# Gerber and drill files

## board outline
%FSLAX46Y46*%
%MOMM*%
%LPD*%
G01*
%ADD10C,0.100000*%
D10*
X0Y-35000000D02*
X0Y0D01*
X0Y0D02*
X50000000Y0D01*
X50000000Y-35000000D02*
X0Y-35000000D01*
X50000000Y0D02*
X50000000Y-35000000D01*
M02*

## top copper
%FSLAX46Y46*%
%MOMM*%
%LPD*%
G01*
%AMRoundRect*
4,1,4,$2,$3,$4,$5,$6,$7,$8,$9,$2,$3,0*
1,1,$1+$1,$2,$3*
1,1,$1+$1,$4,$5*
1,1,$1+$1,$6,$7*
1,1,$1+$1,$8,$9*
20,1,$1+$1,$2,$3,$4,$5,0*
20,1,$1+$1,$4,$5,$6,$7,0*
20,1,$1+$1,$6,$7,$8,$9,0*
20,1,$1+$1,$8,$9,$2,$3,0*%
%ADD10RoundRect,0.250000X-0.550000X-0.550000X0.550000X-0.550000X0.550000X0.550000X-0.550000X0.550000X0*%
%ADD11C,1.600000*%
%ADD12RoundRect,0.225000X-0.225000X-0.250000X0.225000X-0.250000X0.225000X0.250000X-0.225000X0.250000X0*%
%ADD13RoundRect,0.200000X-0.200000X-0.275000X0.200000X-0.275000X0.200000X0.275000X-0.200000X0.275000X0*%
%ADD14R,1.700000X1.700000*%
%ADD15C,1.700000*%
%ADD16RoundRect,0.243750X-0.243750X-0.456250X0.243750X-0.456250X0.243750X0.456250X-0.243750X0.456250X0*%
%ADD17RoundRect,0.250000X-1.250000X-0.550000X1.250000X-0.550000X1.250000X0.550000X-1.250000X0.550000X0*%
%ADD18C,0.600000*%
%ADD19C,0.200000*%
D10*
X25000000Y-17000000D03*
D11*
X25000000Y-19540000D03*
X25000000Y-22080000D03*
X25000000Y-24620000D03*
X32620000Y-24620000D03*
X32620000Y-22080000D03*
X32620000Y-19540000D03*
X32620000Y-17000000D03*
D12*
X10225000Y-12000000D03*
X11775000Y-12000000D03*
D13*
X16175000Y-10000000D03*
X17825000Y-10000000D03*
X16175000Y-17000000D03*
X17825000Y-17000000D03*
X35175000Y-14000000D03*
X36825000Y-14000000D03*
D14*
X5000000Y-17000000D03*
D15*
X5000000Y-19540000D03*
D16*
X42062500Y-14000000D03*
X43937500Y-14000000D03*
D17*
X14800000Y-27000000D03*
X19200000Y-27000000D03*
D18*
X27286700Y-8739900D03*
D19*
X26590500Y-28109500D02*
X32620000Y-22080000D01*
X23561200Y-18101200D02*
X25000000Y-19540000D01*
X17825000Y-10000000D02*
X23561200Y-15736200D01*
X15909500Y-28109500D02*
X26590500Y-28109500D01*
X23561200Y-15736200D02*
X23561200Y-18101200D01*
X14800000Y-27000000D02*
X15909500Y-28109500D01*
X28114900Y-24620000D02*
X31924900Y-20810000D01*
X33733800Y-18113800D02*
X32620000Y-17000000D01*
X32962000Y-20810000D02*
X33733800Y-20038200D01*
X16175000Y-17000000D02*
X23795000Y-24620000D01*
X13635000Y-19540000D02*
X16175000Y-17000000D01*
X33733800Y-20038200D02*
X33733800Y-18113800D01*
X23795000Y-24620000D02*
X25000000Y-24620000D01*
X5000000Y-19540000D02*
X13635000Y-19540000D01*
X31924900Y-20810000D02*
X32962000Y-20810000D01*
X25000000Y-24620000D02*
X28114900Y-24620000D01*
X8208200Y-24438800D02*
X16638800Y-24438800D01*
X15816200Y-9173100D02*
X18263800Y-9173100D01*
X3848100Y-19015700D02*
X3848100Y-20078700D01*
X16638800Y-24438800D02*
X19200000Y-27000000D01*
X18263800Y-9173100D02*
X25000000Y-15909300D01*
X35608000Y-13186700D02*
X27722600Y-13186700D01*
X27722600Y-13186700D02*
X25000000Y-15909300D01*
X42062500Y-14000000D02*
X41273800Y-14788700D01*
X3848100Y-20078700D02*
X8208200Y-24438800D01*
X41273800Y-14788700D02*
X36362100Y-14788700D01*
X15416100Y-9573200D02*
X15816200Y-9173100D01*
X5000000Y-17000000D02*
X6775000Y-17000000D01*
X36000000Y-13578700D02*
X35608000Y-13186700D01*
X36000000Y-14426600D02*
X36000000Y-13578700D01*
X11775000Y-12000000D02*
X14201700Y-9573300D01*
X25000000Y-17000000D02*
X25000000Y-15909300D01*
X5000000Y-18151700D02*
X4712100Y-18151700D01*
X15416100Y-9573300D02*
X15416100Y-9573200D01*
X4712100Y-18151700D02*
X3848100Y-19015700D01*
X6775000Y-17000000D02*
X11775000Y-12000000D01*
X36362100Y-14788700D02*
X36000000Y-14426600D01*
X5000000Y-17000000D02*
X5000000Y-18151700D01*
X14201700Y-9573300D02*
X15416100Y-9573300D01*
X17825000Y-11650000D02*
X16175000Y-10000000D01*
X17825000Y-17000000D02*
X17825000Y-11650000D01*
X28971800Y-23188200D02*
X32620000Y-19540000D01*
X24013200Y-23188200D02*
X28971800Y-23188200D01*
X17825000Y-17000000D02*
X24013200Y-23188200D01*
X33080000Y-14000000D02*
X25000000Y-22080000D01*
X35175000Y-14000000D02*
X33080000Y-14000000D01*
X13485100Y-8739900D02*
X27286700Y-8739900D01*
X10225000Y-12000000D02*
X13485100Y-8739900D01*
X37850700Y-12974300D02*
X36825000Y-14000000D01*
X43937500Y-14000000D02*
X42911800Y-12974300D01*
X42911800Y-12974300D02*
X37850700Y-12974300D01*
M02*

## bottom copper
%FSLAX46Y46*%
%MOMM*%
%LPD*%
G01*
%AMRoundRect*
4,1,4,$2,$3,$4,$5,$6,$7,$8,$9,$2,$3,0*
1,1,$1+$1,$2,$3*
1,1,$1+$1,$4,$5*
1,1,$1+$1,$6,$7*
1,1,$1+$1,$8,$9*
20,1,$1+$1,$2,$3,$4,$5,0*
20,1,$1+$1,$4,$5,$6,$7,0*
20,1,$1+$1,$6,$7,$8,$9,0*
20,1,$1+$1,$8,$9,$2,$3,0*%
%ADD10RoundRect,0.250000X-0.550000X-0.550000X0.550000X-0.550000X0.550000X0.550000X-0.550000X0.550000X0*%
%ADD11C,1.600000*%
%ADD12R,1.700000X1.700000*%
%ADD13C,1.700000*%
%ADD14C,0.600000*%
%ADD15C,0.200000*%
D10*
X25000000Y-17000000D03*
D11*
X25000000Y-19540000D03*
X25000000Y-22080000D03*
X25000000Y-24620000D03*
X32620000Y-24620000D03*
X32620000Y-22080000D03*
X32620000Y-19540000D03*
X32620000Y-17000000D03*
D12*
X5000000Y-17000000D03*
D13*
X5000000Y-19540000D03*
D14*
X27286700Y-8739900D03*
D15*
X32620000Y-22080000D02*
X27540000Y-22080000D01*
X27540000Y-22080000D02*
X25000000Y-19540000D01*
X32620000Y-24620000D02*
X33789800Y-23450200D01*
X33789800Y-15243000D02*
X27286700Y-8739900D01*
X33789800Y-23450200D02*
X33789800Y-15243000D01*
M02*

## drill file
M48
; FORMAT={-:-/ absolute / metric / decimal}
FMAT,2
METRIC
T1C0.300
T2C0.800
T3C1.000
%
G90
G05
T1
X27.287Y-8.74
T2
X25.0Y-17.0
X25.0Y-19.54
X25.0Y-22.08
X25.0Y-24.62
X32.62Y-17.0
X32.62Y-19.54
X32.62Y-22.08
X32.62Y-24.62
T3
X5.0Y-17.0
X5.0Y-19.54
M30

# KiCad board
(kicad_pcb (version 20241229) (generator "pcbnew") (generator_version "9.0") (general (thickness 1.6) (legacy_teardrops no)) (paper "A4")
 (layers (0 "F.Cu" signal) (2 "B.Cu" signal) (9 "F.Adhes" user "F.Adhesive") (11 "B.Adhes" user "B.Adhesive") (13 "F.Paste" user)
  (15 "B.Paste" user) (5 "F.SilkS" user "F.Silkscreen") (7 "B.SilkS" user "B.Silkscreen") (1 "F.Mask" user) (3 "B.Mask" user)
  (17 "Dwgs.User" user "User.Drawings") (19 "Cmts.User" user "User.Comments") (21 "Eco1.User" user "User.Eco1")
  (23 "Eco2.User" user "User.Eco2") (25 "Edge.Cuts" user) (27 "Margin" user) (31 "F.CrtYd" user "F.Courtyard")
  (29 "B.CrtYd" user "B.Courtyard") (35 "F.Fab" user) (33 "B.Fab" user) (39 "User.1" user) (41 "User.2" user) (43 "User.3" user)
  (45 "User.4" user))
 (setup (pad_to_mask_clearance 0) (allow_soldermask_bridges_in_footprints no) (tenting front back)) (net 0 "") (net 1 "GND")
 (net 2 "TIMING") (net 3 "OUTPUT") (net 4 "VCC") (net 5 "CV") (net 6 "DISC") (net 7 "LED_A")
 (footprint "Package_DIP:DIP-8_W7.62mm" (layer "F.Cu") (at 25 17)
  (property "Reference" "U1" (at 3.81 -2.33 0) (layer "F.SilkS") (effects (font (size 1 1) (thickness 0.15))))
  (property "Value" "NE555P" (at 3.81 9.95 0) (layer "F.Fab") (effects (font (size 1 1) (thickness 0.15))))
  (pad "1" thru_hole roundrect (at 0 0) (size 1.6 1.6) (drill 0.8) (layers "*.Cu" "*.Mask") (remove_unused_layers no)
   (roundrect_rratio 0.15625) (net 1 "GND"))
  (pad "2" thru_hole circle (at 0 2.54) (size 1.6 1.6) (drill 0.8) (layers "*.Cu" "*.Mask") (remove_unused_layers no) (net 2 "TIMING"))
  (pad "3" thru_hole circle (at 0 5.08) (size 1.6 1.6) (drill 0.8) (layers "*.Cu" "*.Mask") (remove_unused_layers no) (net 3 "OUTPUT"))
  (pad "4" thru_hole circle (at 0 7.62) (size 1.6 1.6) (drill 0.8) (layers "*.Cu" "*.Mask") (remove_unused_layers no) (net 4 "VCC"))
  (pad "5" thru_hole circle (at 7.62 7.62) (size 1.6 1.6) (drill 0.8) (layers "*.Cu" "*.Mask") (remove_unused_layers no) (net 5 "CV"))
  (pad "6" thru_hole circle (at 7.62 5.08) (size 1.6 1.6) (drill 0.8) (layers "*.Cu" "*.Mask") (remove_unused_layers no) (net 2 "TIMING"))
  (pad "7" thru_hole circle (at 7.62 2.54) (size 1.6 1.6) (drill 0.8) (layers "*.Cu" "*.Mask") (remove_unused_layers no) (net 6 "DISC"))
  (pad "8" thru_hole circle (at 7.62 0) (size 1.6 1.6) (drill 0.8) (layers "*.Cu" "*.Mask") (remove_unused_layers no) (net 4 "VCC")))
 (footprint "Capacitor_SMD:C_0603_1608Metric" (layer "F.Cu") (at 11 12)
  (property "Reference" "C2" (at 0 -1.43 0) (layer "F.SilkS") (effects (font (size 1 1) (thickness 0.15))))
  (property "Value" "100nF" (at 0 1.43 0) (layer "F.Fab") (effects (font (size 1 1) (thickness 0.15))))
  (pad "1" smd roundrect (at -0.775 0) (size 0.9 0.95) (layers "F.Cu" "F.Mask" "F.Paste") (roundrect_rratio 0.25) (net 5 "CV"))
  (pad "2" smd roundrect (at 0.775 0) (size 0.9 0.95) (layers "F.Cu" "F.Mask" "F.Paste") (roundrect_rratio 0.25) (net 1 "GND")))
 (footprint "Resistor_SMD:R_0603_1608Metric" (layer "F.Cu") (at 17 10)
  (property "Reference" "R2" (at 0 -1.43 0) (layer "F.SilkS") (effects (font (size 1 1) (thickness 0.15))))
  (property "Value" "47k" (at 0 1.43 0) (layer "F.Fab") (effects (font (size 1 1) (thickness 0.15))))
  (pad "1" smd roundrect (at -0.825 0) (size 0.8 0.95) (layers "F.Cu" "F.Mask" "F.Paste") (roundrect_rratio 0.25) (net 6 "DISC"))
  (pad "2" smd roundrect (at 0.825 0) (size 0.8 0.95) (layers "F.Cu" "F.Mask" "F.Paste") (roundrect_rratio 0.25) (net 2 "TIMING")))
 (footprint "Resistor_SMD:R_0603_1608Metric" (layer "F.Cu") (at 17 17)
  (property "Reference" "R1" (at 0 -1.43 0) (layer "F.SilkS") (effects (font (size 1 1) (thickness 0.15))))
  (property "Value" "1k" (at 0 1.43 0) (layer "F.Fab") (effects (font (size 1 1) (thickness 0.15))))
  (pad "1" smd roundrect (at -0.825 0) (size 0.8 0.95) (layers "F.Cu" "F.Mask" "F.Paste") (roundrect_rratio 0.25) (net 4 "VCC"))
  (pad "2" smd roundrect (at 0.825 0) (size 0.8 0.95) (layers "F.Cu" "F.Mask" "F.Paste") (roundrect_rratio 0.25) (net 6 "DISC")))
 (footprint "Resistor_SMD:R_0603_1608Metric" (layer "F.Cu") (at 36 14)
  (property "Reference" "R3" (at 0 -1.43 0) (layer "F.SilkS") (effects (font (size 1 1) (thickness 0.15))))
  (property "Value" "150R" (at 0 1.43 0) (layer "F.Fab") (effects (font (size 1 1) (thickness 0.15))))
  (pad "1" smd roundrect (at -0.825 0) (size 0.8 0.95) (layers "F.Cu" "F.Mask" "F.Paste") (roundrect_rratio 0.25) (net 3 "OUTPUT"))
  (pad "2" smd roundrect (at 0.825 0) (size 0.8 0.95) (layers "F.Cu" "F.Mask" "F.Paste") (roundrect_rratio 0.25) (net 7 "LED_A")))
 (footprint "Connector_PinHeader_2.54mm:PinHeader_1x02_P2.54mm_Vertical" (layer "F.Cu") (at 5 17)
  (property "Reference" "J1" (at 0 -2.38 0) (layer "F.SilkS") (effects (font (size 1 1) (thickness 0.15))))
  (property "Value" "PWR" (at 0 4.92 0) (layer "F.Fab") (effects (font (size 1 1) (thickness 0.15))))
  (pad "1" thru_hole rect (at 0 0) (size 1.7 1.7) (drill 1) (layers "*.Cu" "*.Mask") (remove_unused_layers no) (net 1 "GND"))
  (pad "2" thru_hole circle (at 0 2.54) (size 1.7 1.7) (drill 1) (layers "*.Cu" "*.Mask") (remove_unused_layers no) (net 4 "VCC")))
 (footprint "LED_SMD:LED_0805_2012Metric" (layer "F.Cu") (at 43 14)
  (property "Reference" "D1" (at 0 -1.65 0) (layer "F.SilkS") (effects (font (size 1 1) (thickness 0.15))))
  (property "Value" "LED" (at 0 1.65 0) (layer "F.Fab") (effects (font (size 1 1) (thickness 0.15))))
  (pad "1" smd roundrect (at -0.9375 0) (size 0.975 1.4) (layers "F.Cu" "F.Mask" "F.Paste") (roundrect_rratio 0.25) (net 1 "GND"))
  (pad "2" smd roundrect (at 0.9375 0) (size 0.975 1.4) (layers "F.Cu" "F.Mask" "F.Paste") (roundrect_rratio 0.25) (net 7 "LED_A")))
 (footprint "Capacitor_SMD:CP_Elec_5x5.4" (layer "F.Cu") (at 17 27)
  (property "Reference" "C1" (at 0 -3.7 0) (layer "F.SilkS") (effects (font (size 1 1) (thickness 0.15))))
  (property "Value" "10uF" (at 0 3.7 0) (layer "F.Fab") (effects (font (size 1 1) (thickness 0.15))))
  (pad "1" smd roundrect (at -2.2 0) (size 3 1.6) (layers "F.Cu" "F.Mask" "F.Paste") (roundrect_rratio 0.15625) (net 2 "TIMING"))
  (pad "2" smd roundrect (at 2.2 0) (size 3 1.6) (layers "F.Cu" "F.Mask" "F.Paste") (roundrect_rratio 0.15625) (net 1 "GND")))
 (gr_line (start 0 35) (end 0 0) (stroke (width 0.1) (type default)) (layer "Edge.Cuts"))
 (gr_line (start 0 0) (end 50 0) (stroke (width 0.1) (type default)) (layer "Edge.Cuts"))
 (gr_line (start 50 35) (end 0 35) (stroke (width 0.1) (type default)) (layer "Edge.Cuts"))
 (gr_line (start 50 0) (end 50 35) (stroke (width 0.1) (type default)) (layer "Edge.Cuts"))
 (segment (start 26.5905 28.1095) (end 32.62 22.08) (width 0.2) (layer "F.Cu") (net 2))
 (segment (start 23.5612 18.1012) (end 25 19.54) (width 0.2) (layer "F.Cu") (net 2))
 (segment (start 17.825 10) (end 23.5612 15.7362) (width 0.2) (layer "F.Cu") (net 2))
 (segment (start 15.9095 28.1095) (end 26.5905 28.1095) (width 0.2) (layer "F.Cu") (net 2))
 (segment (start 23.5612 15.7362) (end 23.5612 18.1012) (width 0.2) (layer "F.Cu") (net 2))
 (segment (start 14.8 27) (end 15.9095 28.1095) (width 0.2) (layer "F.Cu") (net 2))
 (segment (start 32.62 22.08) (end 27.54 22.08) (width 0.2) (layer "B.Cu") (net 2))
 (segment (start 27.54 22.08) (end 25 19.54) (width 0.2) (layer "B.Cu") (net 2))
 (segment (start 28.1149 24.62) (end 31.9249 20.81) (width 0.2) (layer "F.Cu") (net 4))
 (segment (start 33.7338 18.1138) (end 32.62 17) (width 0.2) (layer "F.Cu") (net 4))
 (segment (start 32.962 20.81) (end 33.7338 20.0382) (width 0.2) (layer "F.Cu") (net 4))
 (segment (start 16.175 17) (end 23.795 24.62) (width 0.2) (layer "F.Cu") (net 4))
 (segment (start 13.635 19.54) (end 16.175 17) (width 0.2) (layer "F.Cu") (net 4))
 (segment (start 33.7338 20.0382) (end 33.7338 18.1138) (width 0.2) (layer "F.Cu") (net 4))
 (segment (start 23.795 24.62) (end 25 24.62) (width 0.2) (layer "F.Cu") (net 4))
 (segment (start 5 19.54) (end 13.635 19.54) (width 0.2) (layer "F.Cu") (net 4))
 (segment (start 31.9249 20.81) (end 32.962 20.81) (width 0.2) (layer "F.Cu") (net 4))
 (segment (start 25 24.62) (end 28.1149 24.62) (width 0.2) (layer "F.Cu") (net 4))
 (segment (start 8.2082 24.4388) (end 16.6388 24.4388) (width 0.2) (layer "F.Cu") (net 1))
 (segment (start 15.8162 9.1731) (end 18.2638 9.1731) (width 0.2) (layer "F.Cu") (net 1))
 (segment (start 3.8481 19.0157) (end 3.8481 20.0787) (width 0.2) (layer "F.Cu") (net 1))
 (segment (start 16.6388 24.4388) (end 19.2 27) (width 0.2) (layer "F.Cu") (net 1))
 (segment (start 18.2638 9.1731) (end 25 15.9093) (width 0.2) (layer "F.Cu") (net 1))
 (segment (start 35.608 13.1867) (end 27.7226 13.1867) (width 0.2) (layer "F.Cu") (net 1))
 (segment (start 27.7226 13.1867) (end 25 15.9093) (width 0.2) (layer "F.Cu") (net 1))
 (segment (start 42.0625 14) (end 41.2738 14.7887) (width 0.2) (layer "F.Cu") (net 1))
 (segment (start 3.8481 20.0787) (end 8.2082 24.4388) (width 0.2) (layer "F.Cu") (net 1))
 (segment (start 41.2738 14.7887) (end 36.3621 14.7887) (width 0.2) (layer "F.Cu") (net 1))
 (segment (start 15.4161 9.5732) (end 15.8162 9.1731) (width 0.2) (layer "F.Cu") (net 1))
 (segment (start 5 17) (end 6.775 17) (width 0.2) (layer "F.Cu") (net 1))
 (segment (start 36 13.5787) (end 35.608 13.1867) (width 0.2) (layer "F.Cu") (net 1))
 (segment (start 36 14.4266) (end 36 13.5787) (width 0.2) (layer "F.Cu") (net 1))
 (segment (start 11.775 12) (end 14.2017 9.5733) (width 0.2) (layer "F.Cu") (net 1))
 (segment (start 25 17) (end 25 15.9093) (width 0.2) (layer "F.Cu") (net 1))
 (segment (start 5 18.1517) (end 4.7121 18.1517) (width 0.2) (layer "F.Cu") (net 1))
 (segment (start 15.4161 9.5733) (end 15.4161 9.5732) (width 0.2) (layer "F.Cu") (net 1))
 (segment (start 4.7121 18.1517) (end 3.8481 19.0157) (width 0.2) (layer "F.Cu") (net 1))
 (segment (start 6.775 17) (end 11.775 12) (width 0.2) (layer "F.Cu") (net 1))
 (segment (start 36.3621 14.7887) (end 36 14.4266) (width 0.2) (layer "F.Cu") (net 1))
 (segment (start 5 17) (end 5 18.1517) (width 0.2) (layer "F.Cu") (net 1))
 (segment (start 14.2017 9.5733) (end 15.4161 9.5733) (width 0.2) (layer "F.Cu") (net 1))
 (segment (start 17.825 11.65) (end 16.175 10) (width 0.2) (layer "F.Cu") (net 6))
 (segment (start 17.825 17) (end 17.825 11.65) (width 0.2) (layer "F.Cu") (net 6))
 (segment (start 28.9718 23.1882) (end 32.62 19.54) (width 0.2) (layer "F.Cu") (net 6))
 (segment (start 24.0132 23.1882) (end 28.9718 23.1882) (width 0.2) (layer "F.Cu") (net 6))
 (segment (start 17.825 17) (end 24.0132 23.1882) (width 0.2) (layer "F.Cu") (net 6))
 (segment (start 33.08 14) (end 25 22.08) (width 0.2) (layer "F.Cu") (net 3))
 (segment (start 35.175 14) (end 33.08 14) (width 0.2) (layer "F.Cu") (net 3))
 (segment (start 13.4851 8.7399) (end 27.2867 8.7399) (width 0.2) (layer "F.Cu") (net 5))
 (segment (start 10.225 12) (end 13.4851 8.7399) (width 0.2) (layer "F.Cu") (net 5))
 (via (at 27.2867 8.7399) (size 0.6) (drill 0.3) (layers "F.Cu" "B.Cu") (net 5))
 (segment (start 32.62 24.62) (end 33.7898 23.4502) (width 0.2) (layer "B.Cu") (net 5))
 (segment (start 33.7898 15.243) (end 27.2867 8.7399) (width 0.2) (layer "B.Cu") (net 5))
 (segment (start 33.7898 23.4502) (end 33.7898 15.243) (width 0.2) (layer "B.Cu") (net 5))
 (segment (start 37.8507 12.9743) (end 36.825 14) (width 0.2) (layer "F.Cu") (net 7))
 (segment (start 43.9375 14) (end 42.9118 12.9743) (width 0.2) (layer "F.Cu") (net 7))
 (segment (start 42.9118 12.9743) (end 37.8507 12.9743) (width 0.2) (layer "F.Cu") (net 7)))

